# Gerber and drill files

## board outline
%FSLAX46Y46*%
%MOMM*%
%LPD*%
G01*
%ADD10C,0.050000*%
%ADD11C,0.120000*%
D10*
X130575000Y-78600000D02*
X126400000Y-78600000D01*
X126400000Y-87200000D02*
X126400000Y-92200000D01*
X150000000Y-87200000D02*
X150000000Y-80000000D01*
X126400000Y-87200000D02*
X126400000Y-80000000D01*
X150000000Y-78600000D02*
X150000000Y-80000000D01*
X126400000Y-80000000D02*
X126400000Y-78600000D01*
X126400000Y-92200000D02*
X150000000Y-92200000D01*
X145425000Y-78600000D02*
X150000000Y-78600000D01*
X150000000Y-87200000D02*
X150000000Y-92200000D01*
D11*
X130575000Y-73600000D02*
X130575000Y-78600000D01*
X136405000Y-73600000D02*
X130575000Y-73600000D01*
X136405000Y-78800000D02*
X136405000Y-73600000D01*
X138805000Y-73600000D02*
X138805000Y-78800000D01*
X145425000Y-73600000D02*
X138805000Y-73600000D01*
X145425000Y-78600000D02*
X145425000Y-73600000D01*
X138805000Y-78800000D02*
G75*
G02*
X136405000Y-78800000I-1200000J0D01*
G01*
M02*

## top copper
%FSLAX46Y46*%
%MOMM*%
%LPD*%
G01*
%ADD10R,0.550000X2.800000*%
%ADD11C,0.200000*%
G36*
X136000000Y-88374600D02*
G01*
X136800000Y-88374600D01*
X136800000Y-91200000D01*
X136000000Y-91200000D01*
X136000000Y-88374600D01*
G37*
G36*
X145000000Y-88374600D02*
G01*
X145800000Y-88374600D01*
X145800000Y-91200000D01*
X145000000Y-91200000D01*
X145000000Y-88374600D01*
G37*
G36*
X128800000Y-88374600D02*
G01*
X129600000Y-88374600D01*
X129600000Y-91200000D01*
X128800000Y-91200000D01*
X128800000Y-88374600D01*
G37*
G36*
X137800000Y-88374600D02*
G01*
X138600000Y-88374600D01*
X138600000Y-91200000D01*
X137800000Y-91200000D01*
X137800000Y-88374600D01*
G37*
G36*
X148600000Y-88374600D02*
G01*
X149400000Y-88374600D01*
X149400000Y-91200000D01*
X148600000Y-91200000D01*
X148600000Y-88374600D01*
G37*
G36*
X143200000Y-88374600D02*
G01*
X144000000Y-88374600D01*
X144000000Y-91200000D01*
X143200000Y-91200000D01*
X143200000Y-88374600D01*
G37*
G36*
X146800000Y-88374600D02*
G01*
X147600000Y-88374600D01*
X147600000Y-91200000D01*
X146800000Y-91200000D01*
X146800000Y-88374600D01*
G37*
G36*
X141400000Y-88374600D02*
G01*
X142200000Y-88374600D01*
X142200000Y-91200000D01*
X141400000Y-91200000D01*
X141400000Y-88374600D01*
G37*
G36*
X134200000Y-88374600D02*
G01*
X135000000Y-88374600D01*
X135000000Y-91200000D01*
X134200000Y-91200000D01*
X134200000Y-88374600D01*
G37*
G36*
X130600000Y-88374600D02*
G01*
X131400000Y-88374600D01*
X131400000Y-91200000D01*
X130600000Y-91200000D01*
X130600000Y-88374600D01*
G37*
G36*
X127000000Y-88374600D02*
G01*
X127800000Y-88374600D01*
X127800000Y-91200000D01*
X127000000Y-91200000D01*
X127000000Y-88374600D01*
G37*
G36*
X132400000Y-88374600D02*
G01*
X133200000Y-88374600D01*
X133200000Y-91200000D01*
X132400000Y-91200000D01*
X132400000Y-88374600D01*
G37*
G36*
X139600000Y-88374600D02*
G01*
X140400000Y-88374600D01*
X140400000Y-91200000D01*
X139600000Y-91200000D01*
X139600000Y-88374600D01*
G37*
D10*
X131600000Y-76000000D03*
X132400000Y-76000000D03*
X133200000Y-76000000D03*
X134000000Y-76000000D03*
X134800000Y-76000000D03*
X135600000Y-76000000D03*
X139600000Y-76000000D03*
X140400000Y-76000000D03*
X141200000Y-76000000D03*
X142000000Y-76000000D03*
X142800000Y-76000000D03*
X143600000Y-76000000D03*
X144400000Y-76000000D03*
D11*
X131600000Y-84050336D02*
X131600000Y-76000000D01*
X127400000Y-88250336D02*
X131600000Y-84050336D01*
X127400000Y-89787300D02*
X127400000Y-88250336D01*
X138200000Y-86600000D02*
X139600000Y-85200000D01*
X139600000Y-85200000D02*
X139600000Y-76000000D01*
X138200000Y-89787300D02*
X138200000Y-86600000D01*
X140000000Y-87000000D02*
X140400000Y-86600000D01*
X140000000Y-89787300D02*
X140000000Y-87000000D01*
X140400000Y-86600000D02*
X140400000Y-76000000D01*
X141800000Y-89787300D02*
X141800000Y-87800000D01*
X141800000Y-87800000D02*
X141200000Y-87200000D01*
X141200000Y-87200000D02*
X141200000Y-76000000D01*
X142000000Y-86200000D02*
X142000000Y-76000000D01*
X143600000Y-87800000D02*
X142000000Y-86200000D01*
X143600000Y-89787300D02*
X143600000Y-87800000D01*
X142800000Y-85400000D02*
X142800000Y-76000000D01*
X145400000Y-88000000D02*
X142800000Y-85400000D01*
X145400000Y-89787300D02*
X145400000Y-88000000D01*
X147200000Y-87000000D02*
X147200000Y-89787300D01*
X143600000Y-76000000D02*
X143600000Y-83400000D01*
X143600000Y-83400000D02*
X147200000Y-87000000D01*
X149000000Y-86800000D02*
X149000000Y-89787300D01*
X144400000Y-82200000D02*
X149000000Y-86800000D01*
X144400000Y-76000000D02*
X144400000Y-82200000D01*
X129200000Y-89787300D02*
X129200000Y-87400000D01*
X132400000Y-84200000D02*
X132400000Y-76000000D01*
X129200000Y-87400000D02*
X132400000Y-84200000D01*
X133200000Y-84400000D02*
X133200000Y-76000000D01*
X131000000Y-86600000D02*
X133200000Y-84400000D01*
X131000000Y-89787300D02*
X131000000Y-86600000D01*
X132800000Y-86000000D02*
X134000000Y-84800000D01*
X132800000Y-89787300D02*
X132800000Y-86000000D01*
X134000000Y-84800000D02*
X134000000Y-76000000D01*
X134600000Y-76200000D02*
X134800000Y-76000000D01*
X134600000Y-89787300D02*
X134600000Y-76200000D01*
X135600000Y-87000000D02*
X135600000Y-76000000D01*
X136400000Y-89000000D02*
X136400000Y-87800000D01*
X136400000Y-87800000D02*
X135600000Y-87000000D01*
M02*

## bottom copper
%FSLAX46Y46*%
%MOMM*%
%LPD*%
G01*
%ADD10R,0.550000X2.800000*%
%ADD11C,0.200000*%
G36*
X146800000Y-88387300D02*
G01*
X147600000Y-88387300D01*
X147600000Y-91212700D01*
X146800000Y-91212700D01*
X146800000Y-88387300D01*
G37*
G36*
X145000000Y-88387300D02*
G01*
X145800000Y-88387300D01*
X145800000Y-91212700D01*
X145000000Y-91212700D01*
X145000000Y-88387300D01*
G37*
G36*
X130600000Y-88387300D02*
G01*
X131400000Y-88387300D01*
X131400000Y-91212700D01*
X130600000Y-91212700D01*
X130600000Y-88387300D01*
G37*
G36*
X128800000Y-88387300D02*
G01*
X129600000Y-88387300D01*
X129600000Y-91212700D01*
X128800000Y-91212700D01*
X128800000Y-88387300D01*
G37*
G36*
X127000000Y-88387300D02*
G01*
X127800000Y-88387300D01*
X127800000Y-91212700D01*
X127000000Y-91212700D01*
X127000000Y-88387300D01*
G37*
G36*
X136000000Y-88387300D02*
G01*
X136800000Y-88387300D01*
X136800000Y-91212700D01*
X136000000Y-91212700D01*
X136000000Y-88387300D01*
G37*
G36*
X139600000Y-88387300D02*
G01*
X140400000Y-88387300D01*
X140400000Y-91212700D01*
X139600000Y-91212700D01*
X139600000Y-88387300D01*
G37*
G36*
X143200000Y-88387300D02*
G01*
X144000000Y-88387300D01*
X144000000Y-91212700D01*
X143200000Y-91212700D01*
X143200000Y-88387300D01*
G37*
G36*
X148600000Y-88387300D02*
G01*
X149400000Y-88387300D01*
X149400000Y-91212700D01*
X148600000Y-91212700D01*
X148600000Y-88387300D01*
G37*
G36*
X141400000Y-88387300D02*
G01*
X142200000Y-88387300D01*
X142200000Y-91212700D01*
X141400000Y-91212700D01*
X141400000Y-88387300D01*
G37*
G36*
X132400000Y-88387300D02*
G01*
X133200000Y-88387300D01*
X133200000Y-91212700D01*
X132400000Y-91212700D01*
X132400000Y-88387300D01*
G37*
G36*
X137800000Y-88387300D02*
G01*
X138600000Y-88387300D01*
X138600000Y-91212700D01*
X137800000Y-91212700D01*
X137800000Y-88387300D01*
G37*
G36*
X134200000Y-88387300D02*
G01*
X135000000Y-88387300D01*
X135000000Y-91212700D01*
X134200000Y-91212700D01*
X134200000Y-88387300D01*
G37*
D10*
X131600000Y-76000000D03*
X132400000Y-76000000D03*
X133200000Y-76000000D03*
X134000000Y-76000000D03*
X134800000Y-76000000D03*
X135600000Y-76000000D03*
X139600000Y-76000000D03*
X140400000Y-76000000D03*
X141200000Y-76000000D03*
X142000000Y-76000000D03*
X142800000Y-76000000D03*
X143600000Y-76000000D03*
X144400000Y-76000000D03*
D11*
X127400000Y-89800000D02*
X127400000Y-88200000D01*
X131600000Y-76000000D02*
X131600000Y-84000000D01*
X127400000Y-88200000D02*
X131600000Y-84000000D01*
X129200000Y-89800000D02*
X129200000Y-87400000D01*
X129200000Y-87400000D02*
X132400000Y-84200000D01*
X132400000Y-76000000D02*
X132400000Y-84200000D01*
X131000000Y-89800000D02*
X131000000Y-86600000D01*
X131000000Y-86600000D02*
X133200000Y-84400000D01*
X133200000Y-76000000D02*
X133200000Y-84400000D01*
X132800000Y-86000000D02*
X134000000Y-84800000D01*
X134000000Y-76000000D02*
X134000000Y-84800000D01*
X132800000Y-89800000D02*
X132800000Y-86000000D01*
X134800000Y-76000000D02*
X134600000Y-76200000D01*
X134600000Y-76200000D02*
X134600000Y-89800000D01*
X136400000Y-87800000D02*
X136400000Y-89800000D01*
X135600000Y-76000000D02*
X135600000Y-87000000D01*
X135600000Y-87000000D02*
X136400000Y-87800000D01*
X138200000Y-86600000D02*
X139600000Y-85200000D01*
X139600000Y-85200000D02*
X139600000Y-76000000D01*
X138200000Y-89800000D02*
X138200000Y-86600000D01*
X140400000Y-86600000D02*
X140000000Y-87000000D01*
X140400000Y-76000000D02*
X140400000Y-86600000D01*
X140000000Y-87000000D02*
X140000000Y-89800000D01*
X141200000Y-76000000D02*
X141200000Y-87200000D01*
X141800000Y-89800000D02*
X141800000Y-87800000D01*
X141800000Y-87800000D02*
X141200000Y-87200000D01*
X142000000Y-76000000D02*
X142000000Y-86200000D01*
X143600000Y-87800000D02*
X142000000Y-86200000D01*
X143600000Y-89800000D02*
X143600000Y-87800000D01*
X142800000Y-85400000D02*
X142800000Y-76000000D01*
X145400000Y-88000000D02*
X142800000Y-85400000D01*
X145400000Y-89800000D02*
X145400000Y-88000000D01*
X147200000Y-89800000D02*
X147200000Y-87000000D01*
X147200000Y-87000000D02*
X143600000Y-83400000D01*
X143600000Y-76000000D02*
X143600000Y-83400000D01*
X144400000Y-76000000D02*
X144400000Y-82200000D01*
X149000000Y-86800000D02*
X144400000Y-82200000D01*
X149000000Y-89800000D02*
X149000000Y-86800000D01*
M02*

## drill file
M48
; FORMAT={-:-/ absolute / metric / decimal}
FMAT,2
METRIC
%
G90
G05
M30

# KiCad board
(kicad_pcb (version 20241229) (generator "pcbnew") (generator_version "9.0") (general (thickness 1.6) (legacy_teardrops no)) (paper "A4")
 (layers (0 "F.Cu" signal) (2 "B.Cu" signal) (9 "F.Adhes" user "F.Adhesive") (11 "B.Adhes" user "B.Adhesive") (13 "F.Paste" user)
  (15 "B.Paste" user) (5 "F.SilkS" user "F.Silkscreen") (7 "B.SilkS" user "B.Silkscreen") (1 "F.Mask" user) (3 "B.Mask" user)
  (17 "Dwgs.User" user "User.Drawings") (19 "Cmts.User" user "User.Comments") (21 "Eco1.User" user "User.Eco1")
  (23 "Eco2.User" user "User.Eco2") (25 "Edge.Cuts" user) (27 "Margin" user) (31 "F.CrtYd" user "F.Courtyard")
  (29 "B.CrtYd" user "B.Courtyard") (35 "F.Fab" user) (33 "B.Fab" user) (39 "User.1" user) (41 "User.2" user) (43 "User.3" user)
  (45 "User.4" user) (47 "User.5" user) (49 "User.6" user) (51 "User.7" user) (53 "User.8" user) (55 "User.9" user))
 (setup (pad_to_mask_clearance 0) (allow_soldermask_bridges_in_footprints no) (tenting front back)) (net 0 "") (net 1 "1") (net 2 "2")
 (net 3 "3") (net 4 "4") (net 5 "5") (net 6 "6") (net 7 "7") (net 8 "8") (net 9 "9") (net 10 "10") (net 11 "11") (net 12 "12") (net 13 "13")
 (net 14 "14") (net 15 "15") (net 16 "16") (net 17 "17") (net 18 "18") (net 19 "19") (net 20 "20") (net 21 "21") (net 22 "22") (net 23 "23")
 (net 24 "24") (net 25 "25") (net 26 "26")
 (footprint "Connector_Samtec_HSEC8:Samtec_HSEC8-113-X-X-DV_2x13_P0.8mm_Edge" (layer "B.Cu") (at 138 73.6)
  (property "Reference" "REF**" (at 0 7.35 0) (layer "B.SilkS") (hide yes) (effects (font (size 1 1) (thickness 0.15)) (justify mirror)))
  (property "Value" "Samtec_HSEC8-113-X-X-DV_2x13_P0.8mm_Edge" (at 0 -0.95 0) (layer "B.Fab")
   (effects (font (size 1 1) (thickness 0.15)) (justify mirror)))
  (fp_line (start -7.425 0) (end -7.425 5) (stroke (width 0.12) (type solid)) (layer "Edge.Cuts"))
  (fp_line (start -1.595 0) (end -7.425 0) (stroke (width 0.12) (type solid)) (layer "Edge.Cuts"))
  (fp_line (start -1.595 5.2) (end -1.595 0) (stroke (width 0.12) (type solid)) (layer "Edge.Cuts"))
  (fp_line (start 0.805 0) (end 0.805 5.2) (stroke (width 0.12) (type solid)) (layer "Edge.Cuts"))
  (fp_line (start 7.425 0) (end 0.805 0) (stroke (width 0.12) (type solid)) (layer "Edge.Cuts"))
  (fp_line (start 7.425 5) (end 7.425 0) (stroke (width 0.12) (type solid)) (layer "Edge.Cuts"))
  (fp_arc (start 0.805 5.2) (mid -0.395 6.4) (end -1.595 5.2) (stroke (width 0.12) (type solid)) (layer "Edge.Cuts"))
  (pad "1" connect rect (at -6.4 2.4) (size 0.55 2.8) (layers "B.Cu" "B.Mask") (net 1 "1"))
  (pad "2" connect rect (at -6.4 2.4) (size 0.55 2.8) (layers "F.Cu" "F.Mask") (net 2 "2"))
  (pad "3" connect rect (at -5.6 2.4) (size 0.55 2.8) (layers "B.Cu" "B.Mask") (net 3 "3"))
  (pad "4" connect rect (at -5.6 2.4) (size 0.55 2.8) (layers "F.Cu" "F.Mask") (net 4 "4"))
  (pad "5" connect rect (at -4.8 2.4) (size 0.55 2.8) (layers "B.Cu" "B.Mask") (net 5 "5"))
  (pad "6" connect rect (at -4.8 2.4) (size 0.55 2.8) (layers "F.Cu" "F.Mask") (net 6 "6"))
  (pad "7" connect rect (at -4 2.4) (size 0.55 2.8) (layers "B.Cu" "B.Mask") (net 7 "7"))
  (pad "8" connect rect (at -4 2.4) (size 0.55 2.8) (layers "F.Cu" "F.Mask") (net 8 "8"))
  (pad "9" connect rect (at -3.2 2.4) (size 0.55 2.8) (layers "B.Cu" "B.Mask") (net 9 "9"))
  (pad "10" connect rect (at -3.2 2.4) (size 0.55 2.8) (layers "F.Cu" "F.Mask") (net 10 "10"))
  (pad "11" connect rect (at -2.4 2.4) (size 0.55 2.8) (layers "B.Cu" "B.Mask") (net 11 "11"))
  (pad "12" connect rect (at -2.4 2.4) (size 0.55 2.8) (layers "F.Cu" "F.Mask") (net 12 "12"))
  (pad "13" connect rect (at 1.6 2.4) (size 0.55 2.8) (layers "B.Cu" "B.Mask") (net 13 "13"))
  (pad "14" connect rect (at 1.6 2.4) (size 0.55 2.8) (layers "F.Cu" "F.Mask") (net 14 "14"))
  (pad "15" connect rect (at 2.4 2.4) (size 0.55 2.8) (layers "B.Cu" "B.Mask") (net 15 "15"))
  (pad "16" connect rect (at 2.4 2.4) (size 0.55 2.8) (layers "F.Cu" "F.Mask") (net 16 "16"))
  (pad "17" connect rect (at 3.2 2.4) (size 0.55 2.8) (layers "B.Cu" "B.Mask") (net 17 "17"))
  (pad "18" connect rect (at 3.2 2.4) (size 0.55 2.8) (layers "F.Cu" "F.Mask") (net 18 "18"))
  (pad "19" connect rect (at 4 2.4) (size 0.55 2.8) (layers "B.Cu" "B.Mask") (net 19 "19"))
  (pad "20" connect rect (at 4 2.4) (size 0.55 2.8) (layers "F.Cu" "F.Mask") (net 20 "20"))
  (pad "21" connect rect (at 4.8 2.4) (size 0.55 2.8) (layers "B.Cu" "B.Mask") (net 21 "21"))
  (pad "22" connect rect (at 4.8 2.4) (size 0.55 2.8) (layers "F.Cu" "F.Mask") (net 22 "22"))
  (pad "23" connect rect (at 5.6 2.4) (size 0.55 2.8) (layers "B.Cu" "B.Mask") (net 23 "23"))
  (pad "24" connect rect (at 5.6 2.4) (size 0.55 2.8) (layers "F.Cu" "F.Mask") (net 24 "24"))
  (pad "25" connect rect (at 6.4 2.4) (size 0.55 2.8) (layers "B.Cu" "B.Mask") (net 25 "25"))
  (pad "26" connect rect (at 6.4 2.4) (size 0.55 2.8) (layers "F.Cu" "F.Mask") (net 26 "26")))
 (gr_rect (start 136 88.3746) (end 136.8 91.2) (stroke (width 0) (type solid)) (fill yes) (layer "F.Cu") (net 12))
 (gr_rect (start 145 88.3746) (end 145.8 91.2) (stroke (width 0) (type solid)) (fill yes) (layer "F.Cu") (net 22))
 (gr_rect (start 128.8 88.3746) (end 129.6 91.2) (stroke (width 0) (type solid)) (fill yes) (layer "F.Cu") (net 4))
 (gr_rect (start 137.8 88.3746) (end 138.6 91.2) (stroke (width 0) (type solid)) (fill yes) (layer "F.Cu") (net 14))
 (gr_rect (start 148.6 88.3746) (end 149.4 91.2) (stroke (width 0) (type solid)) (fill yes) (layer "F.Cu") (net 26))
 (gr_rect (start 143.2 88.3746) (end 144 91.2) (stroke (width 0) (type solid)) (fill yes) (layer "F.Cu") (net 20))
 (gr_rect (start 146.8 88.3746) (end 147.6 91.2) (stroke (width 0) (type solid)) (fill yes) (layer "F.Cu") (net 24))
 (gr_rect (start 141.4 88.3746) (end 142.2 91.2) (stroke (width 0) (type solid)) (fill yes) (layer "F.Cu") (net 18))
 (gr_rect (start 134.2 88.3746) (end 135 91.2) (stroke (width 0) (type solid)) (fill yes) (layer "F.Cu") (net 10))
 (gr_rect (start 130.6 88.3746) (end 131.4 91.2) (stroke (width 0) (type solid)) (fill yes) (layer "F.Cu") (net 6))
 (gr_rect (start 127 88.3746) (end 127.8 91.2) (stroke (width 0) (type solid)) (fill yes) (layer "F.Cu") (net 2))
 (gr_rect (start 132.4 88.3746) (end 133.2 91.2) (stroke (width 0) (type solid)) (fill yes) (layer "F.Cu") (net 8))
 (gr_rect (start 139.6 88.3746) (end 140.4 91.2) (stroke (width 0) (type solid)) (fill yes) (layer "F.Cu") (net 16))
 (gr_rect (start 146.8 88.3873) (end 147.6 91.2127) (stroke (width 0) (type solid)) (fill yes) (layer "B.Cu") (net 23))
 (gr_rect (start 145 88.3873) (end 145.8 91.2127) (stroke (width 0) (type solid)) (fill yes) (layer "B.Cu") (net 21))
 (gr_rect (start 130.6 88.3873) (end 131.4 91.2127) (stroke (width 0) (type solid)) (fill yes) (layer "B.Cu") (net 5))
 (gr_rect (start 128.8 88.3873) (end 129.6 91.2127) (stroke (width 0) (type solid)) (fill yes) (layer "B.Cu") (net 3))
 (gr_rect (start 127 88.3873) (end 127.8 91.2127) (stroke (width 0) (type solid)) (fill yes) (layer "B.Cu") (net 1))
 (gr_rect (start 136 88.3873) (end 136.8 91.2127) (stroke (width 0) (type solid)) (fill yes) (layer "B.Cu") (net 11))
 (gr_rect (start 139.6 88.3873) (end 140.4 91.2127) (stroke (width 0) (type solid)) (fill yes) (layer "B.Cu") (net 15))
 (gr_rect (start 143.2 88.3873) (end 144 91.2127) (stroke (width 0) (type solid)) (fill yes) (layer "B.Cu") (net 19))
 (gr_rect (start 148.6 88.3873) (end 149.4 91.2127) (stroke (width 0) (type solid)) (fill yes) (layer "B.Cu") (net 25))
 (gr_rect (start 141.4 88.3873) (end 142.2 91.2127) (stroke (width 0) (type solid)) (fill yes) (layer "B.Cu") (net 17))
 (gr_rect (start 132.4 88.3873) (end 133.2 91.2127) (stroke (width 0) (type solid)) (fill yes) (layer "B.Cu") (net 7))
 (gr_rect (start 137.8 88.3873) (end 138.6 91.2127) (stroke (width 0) (type solid)) (fill yes) (layer "B.Cu") (net 13))
 (gr_rect (start 134.2 88.3873) (end 135 91.2127) (stroke (width 0) (type solid)) (fill yes) (layer "B.Cu") (net 9))
 (gr_line (start 130.575 78.6) (end 126.4 78.6) (stroke (width 0.05) (type default)) (layer "Edge.Cuts"))
 (gr_line (start 126.4 87.2) (end 126.4 92.2) (stroke (width 0.05) (type default)) (layer "Edge.Cuts"))
 (gr_line (start 150 87.2) (end 150 80) (stroke (width 0.05) (type default)) (layer "Edge.Cuts"))
 (gr_line (start 126.4 87.2) (end 126.4 80) (stroke (width 0.05) (type default)) (layer "Edge.Cuts"))
 (gr_line (start 150 78.6) (end 150 80) (stroke (width 0.05) (type default)) (layer "Edge.Cuts"))
 (gr_line (start 126.4 80) (end 126.4 78.6) (stroke (width 0.05) (type default)) (layer "Edge.Cuts"))
 (gr_line (start 126.4 92.2) (end 150 92.2) (stroke (width 0.05) (type default)) (layer "Edge.Cuts"))
 (gr_line (start 145.425 78.6) (end 150 78.6) (stroke (width 0.05) (type default)) (layer "Edge.Cuts"))
 (gr_line (start 150 87.2) (end 150 92.2) (stroke (width 0.05) (type default)) (layer "Edge.Cuts"))
 (segment (start 131.6 84.050336) (end 131.6 76) (width 0.2) (layer "F.Cu") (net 2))
 (segment (start 127.4 88.250336) (end 131.6 84.050336) (width 0.2) (layer "F.Cu") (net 2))
 (segment (start 127.4 89.7873) (end 127.4 88.250336) (width 0.2) (layer "F.Cu") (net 2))
 (segment (start 127.4 89.8) (end 127.4 88.2) (width 0.2) (layer "B.Cu") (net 1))
 (segment (start 131.6 76) (end 131.6 84) (width 0.2) (layer "B.Cu") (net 1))
 (segment (start 127.4 88.2) (end 131.6 84) (width 0.2) (layer "B.Cu") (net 1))
 (segment (start 138.2 86.6) (end 139.6 85.2) (width 0.2) (layer "F.Cu") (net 14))
 (segment (start 139.6 85.2) (end 139.6 76) (width 0.2) (layer "F.Cu") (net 14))
 (segment (start 138.2 89.7873) (end 138.2 86.6) (width 0.2) (layer "F.Cu") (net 14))
 (segment (start 140 87) (end 140.4 86.6) (width 0.2) (layer "F.Cu") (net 16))
 (segment (start 140 89.7873) (end 140 87) (width 0.2) (layer "F.Cu") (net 16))
 (segment (start 140.4 86.6) (end 140.4 76) (width 0.2) (layer "F.Cu") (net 16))
 (segment (start 141.8 89.7873) (end 141.8 87.8) (width 0.2) (layer "F.Cu") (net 18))
 (segment (start 141.8 87.8) (end 141.2 87.2) (width 0.2) (layer "F.Cu") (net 18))
 (segment (start 141.2 87.2) (end 141.2 76) (width 0.2) (layer "F.Cu") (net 18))
 (segment (start 142 86.2) (end 142 76) (width 0.2) (layer "F.Cu") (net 20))
 (segment (start 143.6 87.8) (end 142 86.2) (width 0.2) (layer "F.Cu") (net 20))
 (segment (start 143.6 89.7873) (end 143.6 87.8) (width 0.2) (layer "F.Cu") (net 20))
 (segment (start 142.8 85.4) (end 142.8 76) (width 0.2) (layer "F.Cu") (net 22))
 (segment (start 145.4 88) (end 142.8 85.4) (width 0.2) (layer "F.Cu") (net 22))
 (segment (start 145.4 89.7873) (end 145.4 88) (width 0.2) (layer "F.Cu") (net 22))
 (segment (start 147.2 87) (end 147.2 89.7873) (width 0.2) (layer "F.Cu") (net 24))
 (segment (start 143.6 76) (end 143.6 83.4) (width 0.2) (layer "F.Cu") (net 24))
 (segment (start 143.6 83.4) (end 147.2 87) (width 0.2) (layer "F.Cu") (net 24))
 (segment (start 149 86.8) (end 149 89.7873) (width 0.2) (layer "F.Cu") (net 26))
 (segment (start 144.4 82.2) (end 149 86.8) (width 0.2) (layer "F.Cu") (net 26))
 (segment (start 144.4 76) (end 144.4 82.2) (width 0.2) (layer "F.Cu") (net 26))
 (segment (start 129.2 89.7873) (end 129.2 87.4) (width 0.2) (layer "F.Cu") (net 4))
 (segment (start 132.4 84.2) (end 132.4 76) (width 0.2) (layer "F.Cu") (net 4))
 (segment (start 129.2 87.4) (end 132.4 84.2) (width 0.2) (layer "F.Cu") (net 4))
 (segment (start 133.2 84.4) (end 133.2 76) (width 0.2) (layer "F.Cu") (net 6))
 (segment (start 131 86.6) (end 133.2 84.4) (width 0.2) (layer "F.Cu") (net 6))
 (segment (start 131 89.7873) (end 131 86.6) (width 0.2) (layer "F.Cu") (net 6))
 (segment (start 132.8 86) (end 134 84.8) (width 0.2) (layer "F.Cu") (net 8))
 (segment (start 132.8 89.7873) (end 132.8 86) (width 0.2) (layer "F.Cu") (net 8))
 (segment (start 134 84.8) (end 134 76) (width 0.2) (layer "F.Cu") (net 8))
 (segment (start 134.6 76.2) (end 134.8 76) (width 0.2) (layer "F.Cu") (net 10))
 (segment (start 134.6 89.7873) (end 134.6 76.2) (width 0.2) (layer "F.Cu") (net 10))
 (segment (start 135.6 87) (end 135.6 76) (width 0.2) (layer "F.Cu") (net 12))
 (segment (start 136.4 89) (end 136.4 87.8) (width 0.2) (layer "F.Cu") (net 12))
 (segment (start 136.4 87.8) (end 135.6 87) (width 0.2) (layer "F.Cu") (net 12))
 (segment (start 129.2 89.8) (end 129.2 87.4) (width 0.2) (layer "B.Cu") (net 3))
 (segment (start 129.2 87.4) (end 132.4 84.2) (width 0.2) (layer "B.Cu") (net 3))
 (segment (start 132.4 76) (end 132.4 84.2) (width 0.2) (layer "B.Cu") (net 3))
 (segment (start 131 89.8) (end 131 86.6) (width 0.2) (layer "B.Cu") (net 5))
 (segment (start 131 86.6) (end 133.2 84.4) (width 0.2) (layer "B.Cu") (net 5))
 (segment (start 133.2 76) (end 133.2 84.4) (width 0.2) (layer "B.Cu") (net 5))
 (segment (start 132.8 86) (end 134 84.8) (width 0.2) (layer "B.Cu") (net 7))
 (segment (start 134 76) (end 134 84.8) (width 0.2) (layer "B.Cu") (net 7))
 (segment (start 132.8 89.8) (end 132.8 86) (width 0.2) (layer "B.Cu") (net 7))
 (segment (start 134.8 76) (end 134.6 76.2) (width 0.2) (layer "B.Cu") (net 9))
 (segment (start 134.6 76.2) (end 134.6 89.8) (width 0.2) (layer "B.Cu") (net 9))
 (segment (start 136.4 87.8) (end 136.4 89.8) (width 0.2) (layer "B.Cu") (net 11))
 (segment (start 135.6 76) (end 135.6 87) (width 0.2) (layer "B.Cu") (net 11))
 (segment (start 135.6 87) (end 136.4 87.8) (width 0.2) (layer "B.Cu") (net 11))
 (segment (start 138.2 86.6) (end 139.6 85.2) (width 0.2) (layer "B.Cu") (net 13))
 (segment (start 139.6 85.2) (end 139.6 76) (width 0.2) (layer "B.Cu") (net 13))
 (segment (start 138.2 89.8) (end 138.2 86.6) (width 0.2) (layer "B.Cu") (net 13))
 (segment (start 140.4 86.6) (end 140 87) (width 0.2) (layer "B.Cu") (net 15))
 (segment (start 140.4 76) (end 140.4 86.6) (width 0.2) (layer "B.Cu") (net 15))
 (segment (start 140 87) (end 140 89.8) (width 0.2) (layer "B.Cu") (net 15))
 (segment (start 141.2 76) (end 141.2 87.2) (width 0.2) (layer "B.Cu") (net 17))
 (segment (start 141.8 89.8) (end 141.8 87.8) (width 0.2) (layer "B.Cu") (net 17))
 (segment (start 141.8 87.8) (end 141.2 87.2) (width 0.2) (layer "B.Cu") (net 17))
 (segment (start 142 76) (end 142 86.2) (width 0.2) (layer "B.Cu") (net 19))
 (segment (start 143.6 87.8) (end 142 86.2) (width 0.2) (layer "B.Cu") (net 19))
 (segment (start 143.6 89.8) (end 143.6 87.8) (width 0.2) (layer "B.Cu") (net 19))
 (segment (start 142.8 85.4) (end 142.8 76) (width 0.2) (layer "B.Cu") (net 21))
 (segment (start 145.4 88) (end 142.8 85.4) (width 0.2) (layer "B.Cu") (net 21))
 (segment (start 145.4 89.8) (end 145.4 88) (width 0.2) (layer "B.Cu") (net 21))
 (segment (start 147.2 89.8) (end 147.2 87) (width 0.2) (layer "B.Cu") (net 23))
 (segment (start 147.2 87) (end 143.6 83.4) (width 0.2) (layer "B.Cu") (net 23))
 (segment (start 143.6 76) (end 143.6 83.4) (width 0.2) (layer "B.Cu") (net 23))
 (segment (start 144.4 76) (end 144.4 82.2) (width 0.2) (layer "B.Cu") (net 25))
 (segment (start 149 86.8) (end 144.4 82.2) (width 0.2) (layer "B.Cu") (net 25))
 (segment (start 149 89.8) (end 149 86.8) (width 0.2) (layer "B.Cu") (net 25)))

